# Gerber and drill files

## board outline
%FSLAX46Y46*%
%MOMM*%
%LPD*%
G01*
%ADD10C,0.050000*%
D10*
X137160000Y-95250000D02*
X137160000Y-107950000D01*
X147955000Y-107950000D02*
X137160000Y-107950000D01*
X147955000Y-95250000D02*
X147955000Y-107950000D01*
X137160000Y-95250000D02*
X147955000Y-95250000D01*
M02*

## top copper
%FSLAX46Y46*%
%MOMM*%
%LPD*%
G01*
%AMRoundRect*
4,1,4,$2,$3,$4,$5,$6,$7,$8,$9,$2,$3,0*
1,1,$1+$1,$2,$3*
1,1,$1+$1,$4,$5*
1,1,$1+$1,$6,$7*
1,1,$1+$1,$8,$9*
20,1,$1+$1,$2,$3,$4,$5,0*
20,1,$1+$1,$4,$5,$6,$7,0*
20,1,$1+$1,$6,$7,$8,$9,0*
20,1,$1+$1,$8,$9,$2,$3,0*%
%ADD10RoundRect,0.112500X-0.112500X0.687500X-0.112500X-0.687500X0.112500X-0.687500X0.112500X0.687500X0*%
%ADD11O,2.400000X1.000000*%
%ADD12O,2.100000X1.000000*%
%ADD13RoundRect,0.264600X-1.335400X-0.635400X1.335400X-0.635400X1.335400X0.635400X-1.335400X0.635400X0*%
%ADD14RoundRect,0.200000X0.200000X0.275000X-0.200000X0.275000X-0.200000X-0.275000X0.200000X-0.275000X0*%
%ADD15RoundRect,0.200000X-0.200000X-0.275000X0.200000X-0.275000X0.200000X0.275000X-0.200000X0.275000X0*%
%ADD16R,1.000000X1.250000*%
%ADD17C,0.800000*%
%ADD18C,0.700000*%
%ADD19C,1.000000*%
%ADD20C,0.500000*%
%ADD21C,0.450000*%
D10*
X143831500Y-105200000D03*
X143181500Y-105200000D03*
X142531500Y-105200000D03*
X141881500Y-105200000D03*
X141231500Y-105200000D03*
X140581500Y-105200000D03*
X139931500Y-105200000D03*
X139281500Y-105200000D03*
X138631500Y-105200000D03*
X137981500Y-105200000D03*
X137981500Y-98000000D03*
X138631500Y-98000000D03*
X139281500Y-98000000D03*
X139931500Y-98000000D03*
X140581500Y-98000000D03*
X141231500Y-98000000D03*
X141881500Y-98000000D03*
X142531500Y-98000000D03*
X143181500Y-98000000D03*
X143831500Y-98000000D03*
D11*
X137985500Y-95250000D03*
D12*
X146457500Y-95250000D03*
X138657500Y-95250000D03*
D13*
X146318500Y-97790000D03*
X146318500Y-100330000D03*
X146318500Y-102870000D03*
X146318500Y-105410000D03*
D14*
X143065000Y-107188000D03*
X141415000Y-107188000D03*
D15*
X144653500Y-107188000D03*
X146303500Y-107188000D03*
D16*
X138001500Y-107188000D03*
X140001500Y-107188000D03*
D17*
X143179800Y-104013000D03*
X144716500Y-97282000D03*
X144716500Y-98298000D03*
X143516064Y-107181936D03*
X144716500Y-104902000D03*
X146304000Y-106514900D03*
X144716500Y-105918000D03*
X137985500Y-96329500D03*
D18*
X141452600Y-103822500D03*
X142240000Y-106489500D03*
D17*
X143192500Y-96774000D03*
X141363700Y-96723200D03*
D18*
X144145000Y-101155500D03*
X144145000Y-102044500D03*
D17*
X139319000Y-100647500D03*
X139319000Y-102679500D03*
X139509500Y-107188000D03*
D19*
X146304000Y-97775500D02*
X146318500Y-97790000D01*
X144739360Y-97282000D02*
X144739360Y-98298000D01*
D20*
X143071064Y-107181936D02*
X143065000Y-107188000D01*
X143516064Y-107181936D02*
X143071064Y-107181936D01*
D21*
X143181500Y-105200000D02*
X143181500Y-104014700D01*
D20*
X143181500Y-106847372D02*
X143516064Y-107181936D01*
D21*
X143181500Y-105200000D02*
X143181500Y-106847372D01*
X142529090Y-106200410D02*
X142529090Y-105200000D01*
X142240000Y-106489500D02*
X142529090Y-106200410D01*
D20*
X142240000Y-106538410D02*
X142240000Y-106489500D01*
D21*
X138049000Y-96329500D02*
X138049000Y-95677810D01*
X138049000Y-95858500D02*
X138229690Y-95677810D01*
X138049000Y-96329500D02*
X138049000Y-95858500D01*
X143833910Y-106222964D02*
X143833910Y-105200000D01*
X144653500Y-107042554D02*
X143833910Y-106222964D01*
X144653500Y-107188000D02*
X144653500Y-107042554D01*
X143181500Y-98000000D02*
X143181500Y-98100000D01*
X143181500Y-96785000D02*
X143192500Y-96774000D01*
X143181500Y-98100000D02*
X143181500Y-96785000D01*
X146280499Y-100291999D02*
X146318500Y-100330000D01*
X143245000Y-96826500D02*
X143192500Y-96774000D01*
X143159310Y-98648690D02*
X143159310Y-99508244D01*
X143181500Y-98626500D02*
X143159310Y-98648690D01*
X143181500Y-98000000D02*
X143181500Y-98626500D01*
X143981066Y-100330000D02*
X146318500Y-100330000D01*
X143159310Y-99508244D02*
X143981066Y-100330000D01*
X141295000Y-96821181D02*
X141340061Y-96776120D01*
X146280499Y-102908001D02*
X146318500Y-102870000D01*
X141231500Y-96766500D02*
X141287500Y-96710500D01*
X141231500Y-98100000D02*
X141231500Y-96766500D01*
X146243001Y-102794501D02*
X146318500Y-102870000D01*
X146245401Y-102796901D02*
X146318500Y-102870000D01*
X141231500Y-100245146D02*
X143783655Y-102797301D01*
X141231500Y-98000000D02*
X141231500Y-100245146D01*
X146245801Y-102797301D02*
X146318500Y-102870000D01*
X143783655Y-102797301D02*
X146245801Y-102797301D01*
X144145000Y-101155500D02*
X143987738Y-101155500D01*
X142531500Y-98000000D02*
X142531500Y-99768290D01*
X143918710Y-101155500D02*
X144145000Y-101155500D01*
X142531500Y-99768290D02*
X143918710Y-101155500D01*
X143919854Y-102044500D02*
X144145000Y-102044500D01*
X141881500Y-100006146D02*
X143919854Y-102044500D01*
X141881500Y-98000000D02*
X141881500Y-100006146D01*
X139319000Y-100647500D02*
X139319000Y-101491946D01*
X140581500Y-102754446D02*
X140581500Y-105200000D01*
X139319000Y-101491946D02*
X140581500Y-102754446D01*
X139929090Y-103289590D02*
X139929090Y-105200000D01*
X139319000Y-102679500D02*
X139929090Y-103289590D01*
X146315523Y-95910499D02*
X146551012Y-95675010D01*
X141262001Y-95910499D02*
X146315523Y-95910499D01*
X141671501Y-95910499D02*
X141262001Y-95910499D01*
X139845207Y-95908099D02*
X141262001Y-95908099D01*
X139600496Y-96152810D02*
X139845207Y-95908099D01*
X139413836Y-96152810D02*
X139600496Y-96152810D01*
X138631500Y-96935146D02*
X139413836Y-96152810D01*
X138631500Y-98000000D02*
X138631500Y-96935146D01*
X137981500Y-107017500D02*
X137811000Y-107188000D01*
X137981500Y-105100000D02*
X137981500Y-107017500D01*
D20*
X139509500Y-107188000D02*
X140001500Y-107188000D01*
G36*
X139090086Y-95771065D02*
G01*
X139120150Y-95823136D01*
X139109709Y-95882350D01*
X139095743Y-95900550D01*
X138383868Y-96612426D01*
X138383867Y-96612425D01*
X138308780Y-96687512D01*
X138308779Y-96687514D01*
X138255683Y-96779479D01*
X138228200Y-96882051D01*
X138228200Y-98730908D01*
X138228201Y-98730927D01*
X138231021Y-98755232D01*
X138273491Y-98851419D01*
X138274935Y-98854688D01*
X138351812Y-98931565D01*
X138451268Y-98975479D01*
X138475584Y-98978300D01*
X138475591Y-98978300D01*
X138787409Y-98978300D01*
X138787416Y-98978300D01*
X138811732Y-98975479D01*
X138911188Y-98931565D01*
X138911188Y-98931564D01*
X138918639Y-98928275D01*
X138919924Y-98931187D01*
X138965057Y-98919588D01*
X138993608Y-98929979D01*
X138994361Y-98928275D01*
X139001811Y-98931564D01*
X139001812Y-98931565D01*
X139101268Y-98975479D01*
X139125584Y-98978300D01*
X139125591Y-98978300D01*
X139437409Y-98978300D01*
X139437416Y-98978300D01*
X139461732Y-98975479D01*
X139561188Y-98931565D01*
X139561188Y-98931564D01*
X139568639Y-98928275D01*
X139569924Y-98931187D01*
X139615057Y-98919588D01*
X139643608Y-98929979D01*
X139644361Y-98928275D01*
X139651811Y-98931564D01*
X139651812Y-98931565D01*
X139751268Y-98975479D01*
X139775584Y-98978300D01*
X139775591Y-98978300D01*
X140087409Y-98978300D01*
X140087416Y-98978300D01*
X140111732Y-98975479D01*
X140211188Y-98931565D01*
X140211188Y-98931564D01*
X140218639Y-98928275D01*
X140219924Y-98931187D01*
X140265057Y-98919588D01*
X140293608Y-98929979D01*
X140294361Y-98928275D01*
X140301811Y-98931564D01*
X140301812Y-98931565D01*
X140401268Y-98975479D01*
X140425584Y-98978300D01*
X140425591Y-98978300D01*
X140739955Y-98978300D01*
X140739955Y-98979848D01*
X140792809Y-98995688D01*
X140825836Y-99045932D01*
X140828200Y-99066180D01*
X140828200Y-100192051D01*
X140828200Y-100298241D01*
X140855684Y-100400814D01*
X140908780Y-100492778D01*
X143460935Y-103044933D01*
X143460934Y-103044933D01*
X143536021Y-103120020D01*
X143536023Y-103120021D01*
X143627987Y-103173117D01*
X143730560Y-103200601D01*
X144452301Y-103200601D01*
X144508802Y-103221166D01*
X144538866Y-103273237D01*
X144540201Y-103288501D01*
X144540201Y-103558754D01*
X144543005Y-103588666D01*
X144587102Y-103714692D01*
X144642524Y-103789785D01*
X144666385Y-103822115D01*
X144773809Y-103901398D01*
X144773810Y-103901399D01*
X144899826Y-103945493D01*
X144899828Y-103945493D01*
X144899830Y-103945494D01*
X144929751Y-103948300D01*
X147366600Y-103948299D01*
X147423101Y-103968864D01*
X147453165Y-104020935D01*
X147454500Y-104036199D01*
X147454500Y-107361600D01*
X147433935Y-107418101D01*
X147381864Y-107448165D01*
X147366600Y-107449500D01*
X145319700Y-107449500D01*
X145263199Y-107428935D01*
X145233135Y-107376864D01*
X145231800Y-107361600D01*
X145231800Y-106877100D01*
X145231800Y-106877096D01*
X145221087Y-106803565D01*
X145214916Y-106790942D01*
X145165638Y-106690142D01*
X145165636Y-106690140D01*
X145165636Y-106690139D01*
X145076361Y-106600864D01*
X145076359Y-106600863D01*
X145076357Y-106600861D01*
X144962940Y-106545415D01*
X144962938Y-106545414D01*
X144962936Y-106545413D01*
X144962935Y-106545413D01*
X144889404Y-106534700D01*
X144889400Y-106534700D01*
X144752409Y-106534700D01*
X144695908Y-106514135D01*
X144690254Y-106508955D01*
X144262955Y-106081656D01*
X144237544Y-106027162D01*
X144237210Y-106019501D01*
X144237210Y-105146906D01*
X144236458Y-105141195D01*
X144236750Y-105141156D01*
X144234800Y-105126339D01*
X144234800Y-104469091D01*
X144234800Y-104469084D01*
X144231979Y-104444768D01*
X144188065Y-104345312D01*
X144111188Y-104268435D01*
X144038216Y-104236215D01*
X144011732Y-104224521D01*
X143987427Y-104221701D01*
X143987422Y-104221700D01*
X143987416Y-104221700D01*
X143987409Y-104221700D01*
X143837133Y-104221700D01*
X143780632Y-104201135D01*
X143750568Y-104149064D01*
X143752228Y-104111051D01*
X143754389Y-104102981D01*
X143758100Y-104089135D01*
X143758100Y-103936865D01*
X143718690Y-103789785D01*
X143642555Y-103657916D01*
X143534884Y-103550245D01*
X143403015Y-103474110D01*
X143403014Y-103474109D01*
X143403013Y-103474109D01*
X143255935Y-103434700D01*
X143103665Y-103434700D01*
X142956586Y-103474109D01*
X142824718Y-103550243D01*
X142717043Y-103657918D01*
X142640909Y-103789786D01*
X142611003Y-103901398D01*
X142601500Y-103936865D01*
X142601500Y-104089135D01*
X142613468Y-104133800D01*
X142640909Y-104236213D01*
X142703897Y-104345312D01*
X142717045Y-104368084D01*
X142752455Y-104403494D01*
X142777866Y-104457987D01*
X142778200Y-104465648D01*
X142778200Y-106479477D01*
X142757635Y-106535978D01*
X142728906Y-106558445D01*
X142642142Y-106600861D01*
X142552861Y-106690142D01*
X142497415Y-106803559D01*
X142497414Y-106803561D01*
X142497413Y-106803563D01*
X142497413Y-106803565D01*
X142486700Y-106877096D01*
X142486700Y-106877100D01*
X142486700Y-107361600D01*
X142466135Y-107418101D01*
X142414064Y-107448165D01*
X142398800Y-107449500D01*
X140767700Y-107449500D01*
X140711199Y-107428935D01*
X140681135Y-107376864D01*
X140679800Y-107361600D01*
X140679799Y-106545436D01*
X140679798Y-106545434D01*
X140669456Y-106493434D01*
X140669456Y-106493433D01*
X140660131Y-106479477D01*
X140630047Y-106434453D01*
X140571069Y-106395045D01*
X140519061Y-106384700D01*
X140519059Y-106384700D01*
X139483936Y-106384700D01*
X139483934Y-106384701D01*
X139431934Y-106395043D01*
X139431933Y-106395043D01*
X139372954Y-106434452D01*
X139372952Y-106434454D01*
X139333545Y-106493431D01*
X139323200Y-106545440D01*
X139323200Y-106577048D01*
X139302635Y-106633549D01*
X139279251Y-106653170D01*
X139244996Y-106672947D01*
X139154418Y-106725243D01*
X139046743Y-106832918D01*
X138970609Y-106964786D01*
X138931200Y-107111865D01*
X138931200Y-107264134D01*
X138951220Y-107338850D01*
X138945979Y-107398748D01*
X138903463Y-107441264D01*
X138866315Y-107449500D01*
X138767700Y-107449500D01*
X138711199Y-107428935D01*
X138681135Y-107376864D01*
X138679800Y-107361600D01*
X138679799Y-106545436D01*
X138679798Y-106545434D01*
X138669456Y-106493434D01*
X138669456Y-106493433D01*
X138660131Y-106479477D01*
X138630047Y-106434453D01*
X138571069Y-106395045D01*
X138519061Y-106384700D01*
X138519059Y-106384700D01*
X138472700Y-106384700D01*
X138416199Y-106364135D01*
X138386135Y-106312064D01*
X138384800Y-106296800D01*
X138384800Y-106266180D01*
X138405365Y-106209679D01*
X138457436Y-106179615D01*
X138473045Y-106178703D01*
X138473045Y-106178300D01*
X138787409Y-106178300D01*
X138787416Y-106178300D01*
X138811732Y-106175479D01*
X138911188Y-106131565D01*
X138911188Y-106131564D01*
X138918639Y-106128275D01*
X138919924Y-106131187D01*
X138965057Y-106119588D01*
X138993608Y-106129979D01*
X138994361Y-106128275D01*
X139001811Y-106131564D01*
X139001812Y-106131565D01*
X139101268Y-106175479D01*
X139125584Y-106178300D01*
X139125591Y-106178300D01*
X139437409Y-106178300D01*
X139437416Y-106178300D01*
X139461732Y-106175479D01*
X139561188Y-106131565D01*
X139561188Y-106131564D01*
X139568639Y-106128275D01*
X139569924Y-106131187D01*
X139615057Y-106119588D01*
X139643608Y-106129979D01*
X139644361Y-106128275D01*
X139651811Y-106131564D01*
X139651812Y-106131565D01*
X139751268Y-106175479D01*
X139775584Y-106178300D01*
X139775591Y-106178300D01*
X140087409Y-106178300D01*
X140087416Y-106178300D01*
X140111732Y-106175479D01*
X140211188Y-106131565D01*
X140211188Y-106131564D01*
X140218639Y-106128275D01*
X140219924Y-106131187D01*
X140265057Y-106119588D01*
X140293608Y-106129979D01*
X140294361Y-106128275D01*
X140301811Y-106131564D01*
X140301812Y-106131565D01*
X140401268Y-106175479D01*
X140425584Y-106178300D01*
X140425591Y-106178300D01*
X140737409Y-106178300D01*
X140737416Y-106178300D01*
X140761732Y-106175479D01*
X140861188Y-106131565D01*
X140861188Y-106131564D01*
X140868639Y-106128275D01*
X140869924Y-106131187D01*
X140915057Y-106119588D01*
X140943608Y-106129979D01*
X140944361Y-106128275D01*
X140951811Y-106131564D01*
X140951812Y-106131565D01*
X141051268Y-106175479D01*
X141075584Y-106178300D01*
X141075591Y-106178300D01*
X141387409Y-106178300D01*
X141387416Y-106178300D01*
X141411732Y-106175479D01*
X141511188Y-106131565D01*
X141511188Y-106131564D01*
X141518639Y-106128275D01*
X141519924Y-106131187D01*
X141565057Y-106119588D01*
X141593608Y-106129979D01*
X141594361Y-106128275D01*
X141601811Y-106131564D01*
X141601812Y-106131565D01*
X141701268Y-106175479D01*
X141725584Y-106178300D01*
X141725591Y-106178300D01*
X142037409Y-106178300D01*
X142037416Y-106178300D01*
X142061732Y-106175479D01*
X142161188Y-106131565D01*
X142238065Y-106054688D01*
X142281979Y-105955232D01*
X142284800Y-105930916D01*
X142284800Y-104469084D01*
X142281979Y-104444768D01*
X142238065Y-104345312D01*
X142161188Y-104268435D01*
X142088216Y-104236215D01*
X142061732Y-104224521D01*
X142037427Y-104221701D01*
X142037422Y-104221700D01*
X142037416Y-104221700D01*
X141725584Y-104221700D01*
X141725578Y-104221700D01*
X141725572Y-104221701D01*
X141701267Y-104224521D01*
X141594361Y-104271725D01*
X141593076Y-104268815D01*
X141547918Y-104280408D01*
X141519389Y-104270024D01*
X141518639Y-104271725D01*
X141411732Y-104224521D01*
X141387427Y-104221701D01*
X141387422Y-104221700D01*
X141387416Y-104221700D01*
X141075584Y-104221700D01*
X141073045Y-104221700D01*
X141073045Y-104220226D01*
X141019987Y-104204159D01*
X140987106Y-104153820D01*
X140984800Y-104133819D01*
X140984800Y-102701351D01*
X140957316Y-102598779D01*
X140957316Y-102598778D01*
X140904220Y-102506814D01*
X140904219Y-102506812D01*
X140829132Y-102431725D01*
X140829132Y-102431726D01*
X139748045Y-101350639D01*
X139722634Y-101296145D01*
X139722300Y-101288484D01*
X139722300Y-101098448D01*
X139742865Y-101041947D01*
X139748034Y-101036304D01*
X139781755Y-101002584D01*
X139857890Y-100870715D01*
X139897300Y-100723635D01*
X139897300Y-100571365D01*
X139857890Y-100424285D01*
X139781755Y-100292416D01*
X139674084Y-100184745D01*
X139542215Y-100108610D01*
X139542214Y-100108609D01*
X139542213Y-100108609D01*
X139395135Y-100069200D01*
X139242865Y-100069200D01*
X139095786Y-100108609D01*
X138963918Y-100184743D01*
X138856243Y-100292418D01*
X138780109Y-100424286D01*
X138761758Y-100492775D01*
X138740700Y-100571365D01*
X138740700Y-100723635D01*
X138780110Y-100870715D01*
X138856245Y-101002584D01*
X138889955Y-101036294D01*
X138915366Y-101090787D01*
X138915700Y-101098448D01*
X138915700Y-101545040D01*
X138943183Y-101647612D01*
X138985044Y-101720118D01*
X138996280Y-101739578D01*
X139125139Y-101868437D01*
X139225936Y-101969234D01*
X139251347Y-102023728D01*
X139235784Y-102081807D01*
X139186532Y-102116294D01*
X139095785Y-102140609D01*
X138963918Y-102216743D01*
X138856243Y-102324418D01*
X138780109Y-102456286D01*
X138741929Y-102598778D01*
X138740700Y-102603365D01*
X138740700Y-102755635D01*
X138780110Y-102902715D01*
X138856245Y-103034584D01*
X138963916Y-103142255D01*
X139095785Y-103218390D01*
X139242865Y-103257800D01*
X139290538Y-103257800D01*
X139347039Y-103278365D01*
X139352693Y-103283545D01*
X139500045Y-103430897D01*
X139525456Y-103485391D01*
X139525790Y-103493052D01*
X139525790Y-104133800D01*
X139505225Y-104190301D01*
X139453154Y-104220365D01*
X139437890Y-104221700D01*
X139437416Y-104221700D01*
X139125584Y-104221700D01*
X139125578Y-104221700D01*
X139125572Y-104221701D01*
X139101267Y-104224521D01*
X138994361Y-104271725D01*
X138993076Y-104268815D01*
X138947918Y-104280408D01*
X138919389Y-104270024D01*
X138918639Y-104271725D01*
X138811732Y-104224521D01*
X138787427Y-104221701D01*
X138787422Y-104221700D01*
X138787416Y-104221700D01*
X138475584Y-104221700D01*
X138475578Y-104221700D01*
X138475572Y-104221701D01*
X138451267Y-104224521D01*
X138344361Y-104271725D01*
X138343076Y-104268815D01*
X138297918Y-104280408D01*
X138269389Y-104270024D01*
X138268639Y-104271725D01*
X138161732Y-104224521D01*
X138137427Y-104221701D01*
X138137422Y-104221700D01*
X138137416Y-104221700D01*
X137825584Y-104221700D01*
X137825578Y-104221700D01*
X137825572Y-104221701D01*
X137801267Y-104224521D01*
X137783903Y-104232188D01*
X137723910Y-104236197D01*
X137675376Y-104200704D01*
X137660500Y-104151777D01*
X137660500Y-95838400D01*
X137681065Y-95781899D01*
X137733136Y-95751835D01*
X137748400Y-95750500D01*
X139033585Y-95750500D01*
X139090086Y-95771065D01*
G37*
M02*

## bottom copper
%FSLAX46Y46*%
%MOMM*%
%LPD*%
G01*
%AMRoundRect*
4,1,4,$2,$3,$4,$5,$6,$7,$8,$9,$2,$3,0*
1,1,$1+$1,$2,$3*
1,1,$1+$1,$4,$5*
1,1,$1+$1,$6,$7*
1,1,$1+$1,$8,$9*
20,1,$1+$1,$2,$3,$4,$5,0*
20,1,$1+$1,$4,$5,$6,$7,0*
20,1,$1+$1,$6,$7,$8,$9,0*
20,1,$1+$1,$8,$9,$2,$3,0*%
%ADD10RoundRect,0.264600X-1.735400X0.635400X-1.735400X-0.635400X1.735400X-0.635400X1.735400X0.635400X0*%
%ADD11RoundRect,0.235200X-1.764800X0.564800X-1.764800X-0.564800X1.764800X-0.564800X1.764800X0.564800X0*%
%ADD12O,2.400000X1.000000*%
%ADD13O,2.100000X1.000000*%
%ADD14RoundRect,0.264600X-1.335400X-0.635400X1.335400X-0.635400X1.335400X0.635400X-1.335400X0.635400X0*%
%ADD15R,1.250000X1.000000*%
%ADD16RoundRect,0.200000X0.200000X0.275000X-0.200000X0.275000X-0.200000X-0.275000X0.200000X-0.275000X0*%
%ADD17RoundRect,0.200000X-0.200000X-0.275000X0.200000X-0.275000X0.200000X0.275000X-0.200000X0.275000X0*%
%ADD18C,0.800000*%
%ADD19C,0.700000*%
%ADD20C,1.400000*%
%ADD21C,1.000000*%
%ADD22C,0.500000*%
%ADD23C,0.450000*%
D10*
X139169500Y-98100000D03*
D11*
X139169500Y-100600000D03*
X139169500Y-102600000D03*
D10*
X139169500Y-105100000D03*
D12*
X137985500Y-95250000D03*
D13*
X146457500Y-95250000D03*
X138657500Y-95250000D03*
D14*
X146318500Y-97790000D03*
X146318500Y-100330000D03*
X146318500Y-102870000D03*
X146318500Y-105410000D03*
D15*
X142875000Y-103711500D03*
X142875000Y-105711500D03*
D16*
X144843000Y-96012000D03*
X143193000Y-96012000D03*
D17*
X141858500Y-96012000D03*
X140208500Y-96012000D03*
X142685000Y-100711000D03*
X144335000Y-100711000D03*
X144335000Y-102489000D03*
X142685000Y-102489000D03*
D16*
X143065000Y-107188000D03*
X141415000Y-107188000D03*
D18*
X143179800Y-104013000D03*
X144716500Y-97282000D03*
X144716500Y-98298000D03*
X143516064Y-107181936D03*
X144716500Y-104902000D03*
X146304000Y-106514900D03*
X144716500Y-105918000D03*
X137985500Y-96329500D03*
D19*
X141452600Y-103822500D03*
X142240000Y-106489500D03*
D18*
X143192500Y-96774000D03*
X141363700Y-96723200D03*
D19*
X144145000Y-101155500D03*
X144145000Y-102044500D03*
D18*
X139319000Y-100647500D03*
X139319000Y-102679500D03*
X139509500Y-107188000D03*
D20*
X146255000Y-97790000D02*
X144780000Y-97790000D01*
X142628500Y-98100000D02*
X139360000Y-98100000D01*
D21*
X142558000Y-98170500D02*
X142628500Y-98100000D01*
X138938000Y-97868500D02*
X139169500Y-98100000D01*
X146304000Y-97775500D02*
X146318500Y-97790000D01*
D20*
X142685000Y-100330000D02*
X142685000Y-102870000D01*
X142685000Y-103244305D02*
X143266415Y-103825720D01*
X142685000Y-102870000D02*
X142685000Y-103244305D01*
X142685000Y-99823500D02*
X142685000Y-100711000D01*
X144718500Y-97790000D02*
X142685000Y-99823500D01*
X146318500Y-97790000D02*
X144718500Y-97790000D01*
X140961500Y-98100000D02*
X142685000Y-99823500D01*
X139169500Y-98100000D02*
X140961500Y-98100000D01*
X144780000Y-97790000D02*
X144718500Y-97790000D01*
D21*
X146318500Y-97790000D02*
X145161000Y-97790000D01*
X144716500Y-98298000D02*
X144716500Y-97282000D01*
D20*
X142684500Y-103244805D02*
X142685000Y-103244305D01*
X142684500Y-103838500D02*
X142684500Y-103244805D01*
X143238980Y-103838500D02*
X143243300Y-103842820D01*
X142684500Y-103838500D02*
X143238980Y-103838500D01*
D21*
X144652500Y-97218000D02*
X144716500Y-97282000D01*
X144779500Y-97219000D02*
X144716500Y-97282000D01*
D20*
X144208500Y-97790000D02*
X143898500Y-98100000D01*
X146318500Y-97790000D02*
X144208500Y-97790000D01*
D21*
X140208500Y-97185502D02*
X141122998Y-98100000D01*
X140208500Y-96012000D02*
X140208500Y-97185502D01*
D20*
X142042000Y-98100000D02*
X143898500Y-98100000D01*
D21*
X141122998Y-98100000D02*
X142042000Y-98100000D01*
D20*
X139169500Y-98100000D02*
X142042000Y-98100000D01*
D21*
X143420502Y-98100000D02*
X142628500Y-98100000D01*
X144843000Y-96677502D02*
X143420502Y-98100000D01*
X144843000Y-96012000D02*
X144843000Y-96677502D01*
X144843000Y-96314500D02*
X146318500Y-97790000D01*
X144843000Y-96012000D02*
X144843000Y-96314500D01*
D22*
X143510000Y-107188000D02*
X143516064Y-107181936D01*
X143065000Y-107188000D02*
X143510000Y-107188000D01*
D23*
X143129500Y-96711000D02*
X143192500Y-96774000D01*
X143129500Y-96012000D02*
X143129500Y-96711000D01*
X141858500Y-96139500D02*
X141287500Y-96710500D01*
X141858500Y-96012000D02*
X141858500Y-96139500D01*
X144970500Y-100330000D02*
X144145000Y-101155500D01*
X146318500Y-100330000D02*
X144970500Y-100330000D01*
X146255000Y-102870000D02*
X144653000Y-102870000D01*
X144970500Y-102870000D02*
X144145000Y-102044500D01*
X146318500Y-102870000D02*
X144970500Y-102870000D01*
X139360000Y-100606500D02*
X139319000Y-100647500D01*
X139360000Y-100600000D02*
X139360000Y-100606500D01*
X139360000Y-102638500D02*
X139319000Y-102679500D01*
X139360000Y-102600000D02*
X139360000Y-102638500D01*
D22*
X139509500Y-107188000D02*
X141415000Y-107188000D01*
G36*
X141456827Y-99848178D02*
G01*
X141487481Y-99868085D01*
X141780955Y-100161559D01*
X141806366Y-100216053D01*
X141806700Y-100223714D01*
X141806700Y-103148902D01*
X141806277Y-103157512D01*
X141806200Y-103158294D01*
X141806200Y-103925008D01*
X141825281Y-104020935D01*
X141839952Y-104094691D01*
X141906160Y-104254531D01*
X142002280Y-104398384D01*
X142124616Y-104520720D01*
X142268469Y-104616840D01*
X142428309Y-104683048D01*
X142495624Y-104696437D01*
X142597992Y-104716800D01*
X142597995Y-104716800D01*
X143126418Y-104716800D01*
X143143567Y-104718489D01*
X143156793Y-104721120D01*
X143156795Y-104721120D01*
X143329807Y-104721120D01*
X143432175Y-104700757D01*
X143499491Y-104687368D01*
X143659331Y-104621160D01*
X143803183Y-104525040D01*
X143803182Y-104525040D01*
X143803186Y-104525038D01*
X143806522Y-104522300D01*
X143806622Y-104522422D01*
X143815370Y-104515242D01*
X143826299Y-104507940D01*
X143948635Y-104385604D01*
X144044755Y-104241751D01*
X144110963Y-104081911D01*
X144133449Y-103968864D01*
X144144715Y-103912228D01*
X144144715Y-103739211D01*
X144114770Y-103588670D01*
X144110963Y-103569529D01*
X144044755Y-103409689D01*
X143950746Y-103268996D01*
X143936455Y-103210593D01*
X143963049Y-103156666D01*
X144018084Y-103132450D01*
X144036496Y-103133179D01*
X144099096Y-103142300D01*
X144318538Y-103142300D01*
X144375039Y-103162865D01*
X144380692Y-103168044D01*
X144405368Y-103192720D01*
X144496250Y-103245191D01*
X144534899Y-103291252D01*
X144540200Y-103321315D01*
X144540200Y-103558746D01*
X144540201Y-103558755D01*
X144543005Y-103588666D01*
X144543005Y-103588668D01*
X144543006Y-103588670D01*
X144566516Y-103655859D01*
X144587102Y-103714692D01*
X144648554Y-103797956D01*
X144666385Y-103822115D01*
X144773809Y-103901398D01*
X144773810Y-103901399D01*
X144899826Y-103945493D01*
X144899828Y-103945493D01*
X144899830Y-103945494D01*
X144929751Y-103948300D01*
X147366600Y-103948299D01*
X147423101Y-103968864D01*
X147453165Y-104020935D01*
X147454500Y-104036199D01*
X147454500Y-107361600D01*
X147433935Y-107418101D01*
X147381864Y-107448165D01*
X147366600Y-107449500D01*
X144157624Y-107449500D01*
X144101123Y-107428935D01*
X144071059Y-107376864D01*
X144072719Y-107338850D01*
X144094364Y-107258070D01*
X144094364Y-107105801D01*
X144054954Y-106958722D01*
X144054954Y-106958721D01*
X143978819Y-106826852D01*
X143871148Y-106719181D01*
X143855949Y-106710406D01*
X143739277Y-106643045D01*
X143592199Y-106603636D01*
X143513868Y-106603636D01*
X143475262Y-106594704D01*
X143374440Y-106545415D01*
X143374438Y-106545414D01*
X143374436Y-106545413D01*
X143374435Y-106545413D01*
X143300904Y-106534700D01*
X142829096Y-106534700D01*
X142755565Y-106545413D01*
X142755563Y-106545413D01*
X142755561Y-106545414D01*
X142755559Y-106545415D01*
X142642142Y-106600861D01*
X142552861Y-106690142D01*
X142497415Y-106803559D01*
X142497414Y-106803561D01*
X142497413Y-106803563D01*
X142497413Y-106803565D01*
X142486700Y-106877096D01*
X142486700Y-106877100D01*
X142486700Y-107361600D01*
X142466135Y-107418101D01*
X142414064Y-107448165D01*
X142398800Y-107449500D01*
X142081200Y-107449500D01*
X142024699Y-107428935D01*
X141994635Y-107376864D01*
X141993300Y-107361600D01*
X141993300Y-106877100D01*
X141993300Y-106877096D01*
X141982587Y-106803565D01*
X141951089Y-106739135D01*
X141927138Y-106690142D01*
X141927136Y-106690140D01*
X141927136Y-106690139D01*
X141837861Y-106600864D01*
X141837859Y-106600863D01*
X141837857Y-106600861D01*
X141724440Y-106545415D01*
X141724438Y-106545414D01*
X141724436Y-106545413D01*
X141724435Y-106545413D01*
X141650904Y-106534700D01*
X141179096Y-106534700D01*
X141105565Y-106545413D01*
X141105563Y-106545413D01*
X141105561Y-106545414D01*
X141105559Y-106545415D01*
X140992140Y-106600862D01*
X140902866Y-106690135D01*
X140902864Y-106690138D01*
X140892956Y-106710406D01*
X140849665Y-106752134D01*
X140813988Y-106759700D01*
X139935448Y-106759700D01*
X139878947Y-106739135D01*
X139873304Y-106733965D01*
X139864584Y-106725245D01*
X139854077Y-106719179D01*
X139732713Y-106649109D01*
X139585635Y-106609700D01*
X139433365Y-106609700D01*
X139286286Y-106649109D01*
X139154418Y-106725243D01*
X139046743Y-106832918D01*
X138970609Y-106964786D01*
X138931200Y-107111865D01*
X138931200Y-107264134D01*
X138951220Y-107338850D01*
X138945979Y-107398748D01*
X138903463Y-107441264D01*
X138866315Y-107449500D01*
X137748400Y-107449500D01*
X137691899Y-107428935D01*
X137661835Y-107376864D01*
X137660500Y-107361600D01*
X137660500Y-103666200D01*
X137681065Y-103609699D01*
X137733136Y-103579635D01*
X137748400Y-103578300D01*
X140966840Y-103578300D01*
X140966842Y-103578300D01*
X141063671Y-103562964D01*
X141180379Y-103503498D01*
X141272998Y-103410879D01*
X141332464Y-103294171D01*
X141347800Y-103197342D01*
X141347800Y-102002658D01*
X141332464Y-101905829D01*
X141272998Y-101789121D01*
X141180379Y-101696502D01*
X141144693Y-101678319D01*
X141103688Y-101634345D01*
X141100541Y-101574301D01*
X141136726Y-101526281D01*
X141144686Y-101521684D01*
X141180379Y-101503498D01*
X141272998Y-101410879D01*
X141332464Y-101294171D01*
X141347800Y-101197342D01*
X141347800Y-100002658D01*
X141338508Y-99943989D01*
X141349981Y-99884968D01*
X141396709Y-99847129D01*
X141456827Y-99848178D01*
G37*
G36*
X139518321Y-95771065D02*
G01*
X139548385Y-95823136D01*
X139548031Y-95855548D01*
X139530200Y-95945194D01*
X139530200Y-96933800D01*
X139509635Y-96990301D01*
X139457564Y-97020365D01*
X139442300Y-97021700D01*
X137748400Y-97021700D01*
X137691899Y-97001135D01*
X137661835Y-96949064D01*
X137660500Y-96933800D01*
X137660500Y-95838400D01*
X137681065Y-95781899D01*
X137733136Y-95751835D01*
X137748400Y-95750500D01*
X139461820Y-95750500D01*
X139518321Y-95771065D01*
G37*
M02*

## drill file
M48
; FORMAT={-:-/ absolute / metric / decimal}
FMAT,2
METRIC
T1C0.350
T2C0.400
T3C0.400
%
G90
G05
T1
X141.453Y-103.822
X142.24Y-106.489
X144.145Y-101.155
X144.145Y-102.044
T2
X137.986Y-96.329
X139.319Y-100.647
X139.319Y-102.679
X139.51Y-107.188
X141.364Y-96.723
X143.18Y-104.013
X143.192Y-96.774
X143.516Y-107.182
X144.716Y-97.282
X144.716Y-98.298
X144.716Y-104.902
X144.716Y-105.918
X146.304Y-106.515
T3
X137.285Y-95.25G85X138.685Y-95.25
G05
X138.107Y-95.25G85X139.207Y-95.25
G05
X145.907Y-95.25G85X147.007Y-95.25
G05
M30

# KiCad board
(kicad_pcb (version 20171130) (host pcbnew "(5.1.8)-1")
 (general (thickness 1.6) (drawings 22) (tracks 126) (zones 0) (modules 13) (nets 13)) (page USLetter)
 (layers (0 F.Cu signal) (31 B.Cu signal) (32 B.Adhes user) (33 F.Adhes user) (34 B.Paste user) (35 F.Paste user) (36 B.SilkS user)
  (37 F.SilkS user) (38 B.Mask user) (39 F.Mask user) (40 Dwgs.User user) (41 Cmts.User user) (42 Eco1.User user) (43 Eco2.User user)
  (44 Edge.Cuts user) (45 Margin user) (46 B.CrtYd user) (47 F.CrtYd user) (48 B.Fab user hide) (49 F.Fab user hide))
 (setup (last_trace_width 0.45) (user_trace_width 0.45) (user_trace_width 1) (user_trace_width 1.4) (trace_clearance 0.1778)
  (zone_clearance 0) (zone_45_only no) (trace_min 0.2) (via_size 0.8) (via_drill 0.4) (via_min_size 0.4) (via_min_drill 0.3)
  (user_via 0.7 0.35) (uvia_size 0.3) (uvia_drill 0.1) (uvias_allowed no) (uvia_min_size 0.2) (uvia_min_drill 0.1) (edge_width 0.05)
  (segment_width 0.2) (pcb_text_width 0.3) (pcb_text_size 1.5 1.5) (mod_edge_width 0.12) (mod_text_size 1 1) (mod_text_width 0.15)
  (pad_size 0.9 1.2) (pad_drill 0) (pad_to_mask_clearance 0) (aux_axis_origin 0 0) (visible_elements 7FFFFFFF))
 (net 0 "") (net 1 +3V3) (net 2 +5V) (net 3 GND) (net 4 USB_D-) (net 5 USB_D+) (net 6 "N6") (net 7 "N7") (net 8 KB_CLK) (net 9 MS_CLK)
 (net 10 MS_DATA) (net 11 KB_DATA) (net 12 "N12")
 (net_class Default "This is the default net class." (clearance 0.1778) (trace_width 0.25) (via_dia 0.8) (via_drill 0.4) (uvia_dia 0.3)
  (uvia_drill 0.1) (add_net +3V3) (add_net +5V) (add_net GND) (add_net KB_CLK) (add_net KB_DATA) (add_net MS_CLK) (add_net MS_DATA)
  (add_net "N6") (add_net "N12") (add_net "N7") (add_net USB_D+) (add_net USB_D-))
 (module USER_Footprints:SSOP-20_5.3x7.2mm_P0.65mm (layer F.Cu) (at 140.9065 101.6 270)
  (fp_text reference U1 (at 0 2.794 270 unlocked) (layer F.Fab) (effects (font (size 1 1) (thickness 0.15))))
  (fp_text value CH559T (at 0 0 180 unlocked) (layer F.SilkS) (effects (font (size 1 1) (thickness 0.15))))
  (pad 20 smd roundrect (at 3.6 -2.925 270) (size 1.6 0.45) (layers F.Cu F.Paste F.Mask) (roundrect_rratio 0.25) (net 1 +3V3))
  (pad 19 smd roundrect (at 3.6 -2.275 270) (size 1.6 0.45) (layers F.Cu F.Paste F.Mask) (roundrect_rratio 0.25) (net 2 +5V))
  (pad 18 smd roundrect (at 3.6 -1.625 270) (size 1.6 0.45) (layers F.Cu F.Paste F.Mask) (roundrect_rratio 0.25) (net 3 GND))
  (pad 17 smd roundrect (at 3.6 -0.975 270) (size 1.6 0.45) (layers F.Cu F.Paste F.Mask) (roundrect_rratio 0.25))
  (pad 16 smd roundrect (at 3.6 -0.325 270) (size 1.6 0.45) (layers F.Cu F.Paste F.Mask) (roundrect_rratio 0.25))
  (pad 15 smd roundrect (at 3.6 0.325 270) (size 1.6 0.45) (layers F.Cu F.Paste F.Mask) (roundrect_rratio 0.25) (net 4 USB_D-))
  (pad 14 smd roundrect (at 3.6 0.975 270) (size 1.6 0.45) (layers F.Cu F.Paste F.Mask) (roundrect_rratio 0.25) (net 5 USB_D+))
  (pad 13 smd roundrect (at 3.6 1.625 270) (size 1.6 0.45) (layers F.Cu F.Paste F.Mask) (roundrect_rratio 0.25))
  (pad 12 smd roundrect (at 3.6 2.275 270) (size 1.6 0.45) (layers F.Cu F.Paste F.Mask) (roundrect_rratio 0.25))
  (pad 11 smd roundrect (at 3.6 2.925 270) (size 1.6 0.45) (layers F.Cu F.Paste F.Mask) (roundrect_rratio 0.25) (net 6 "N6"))
  (pad 10 smd roundrect (at -3.6 2.925 270) (size 1.6 0.45) (layers F.Cu F.Paste F.Mask) (roundrect_rratio 0.25) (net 3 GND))
  (pad 9 smd roundrect (at -3.6 2.275 270) (size 1.6 0.45) (layers F.Cu F.Paste F.Mask) (roundrect_rratio 0.25) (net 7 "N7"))
  (pad 8 smd roundrect (at -3.6 1.625 270) (size 1.6 0.45) (layers F.Cu F.Paste F.Mask) (roundrect_rratio 0.25))
  (pad 7 smd roundrect (at -3.6 0.975 270) (size 1.6 0.45) (layers F.Cu F.Paste F.Mask) (roundrect_rratio 0.25))
  (pad 6 smd roundrect (at -3.6 0.325 270) (size 1.6 0.45) (layers F.Cu F.Paste F.Mask) (roundrect_rratio 0.25))
  (pad 5 smd roundrect (at -3.6 -0.325 270) (size 1.6 0.45) (layers F.Cu F.Paste F.Mask) (roundrect_rratio 0.25) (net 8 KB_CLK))
  (pad 4 smd roundrect (at -3.6 -0.975 270) (size 1.6 0.45) (layers F.Cu F.Paste F.Mask) (roundrect_rratio 0.25) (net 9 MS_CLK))
  (pad 3 smd roundrect (at -3.6 -1.625 270) (size 1.6 0.45) (layers F.Cu F.Paste F.Mask) (roundrect_rratio 0.25) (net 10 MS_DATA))
  (pad 2 smd roundrect (at -3.6 -2.275 270) (size 1.6 0.45) (layers F.Cu F.Paste F.Mask) (roundrect_rratio 0.25) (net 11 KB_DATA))
  (pad 1 smd roundrect (at -3.6 -2.925 270) (size 1.6 0.45) (layers F.Cu F.Paste F.Mask) (roundrect_rratio 0.25)))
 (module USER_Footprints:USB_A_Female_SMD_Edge (layer F.Cu) (at 136.9695 101.6 270)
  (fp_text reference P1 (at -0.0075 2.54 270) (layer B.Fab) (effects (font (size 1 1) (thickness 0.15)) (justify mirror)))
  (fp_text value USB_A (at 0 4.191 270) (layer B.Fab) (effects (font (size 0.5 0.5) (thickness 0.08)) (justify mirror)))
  (pad 1 smd roundrect (at -3.5 -2.2 270) (size 1.8 4) (layers B.Cu B.Paste B.Mask) (roundrect_rratio 0.147) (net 2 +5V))
  (pad 2 smd roundrect (at -1 -2.2 270) (size 1.6 4) (layers B.Cu B.Paste B.Mask) (roundrect_rratio 0.147) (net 4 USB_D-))
  (pad 3 smd roundrect (at 1 -2.2 270) (size 1.6 4) (layers B.Cu B.Paste B.Mask) (roundrect_rratio 0.147) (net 5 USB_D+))
  (pad 4 smd roundrect (at 3.5 -2.2 270) (size 1.8 4) (layers B.Cu B.Paste B.Mask) (roundrect_rratio 0.147) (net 3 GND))
  (pad 4 thru_hole oval (at -6.35 -1.016) (size 2.4 1) (drill oval 1.8 0.4) (layers *.Cu *.Mask) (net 3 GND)))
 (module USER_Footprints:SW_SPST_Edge (layer F.Cu) (at 142.5575 95.25)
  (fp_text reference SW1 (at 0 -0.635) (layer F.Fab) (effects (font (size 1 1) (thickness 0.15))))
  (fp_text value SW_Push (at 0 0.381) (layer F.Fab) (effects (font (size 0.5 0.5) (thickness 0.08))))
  (pad 2 thru_hole oval (at 3.9 0) (size 2.1 1) (drill oval 1.5 0.4) (layers *.Cu *.Mask) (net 7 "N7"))
  (pad 1 thru_hole oval (at -3.9 0) (size 2.1 1) (drill oval 1.5 0.4) (layers *.Cu *.Mask) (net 3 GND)))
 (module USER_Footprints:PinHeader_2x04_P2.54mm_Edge (layer F.Cu) (at 148.0185 97.79)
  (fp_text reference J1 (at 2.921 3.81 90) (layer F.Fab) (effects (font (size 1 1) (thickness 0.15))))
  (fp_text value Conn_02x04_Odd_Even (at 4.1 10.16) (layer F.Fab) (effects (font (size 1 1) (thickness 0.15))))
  (pad 1 smd roundrect (at -1.7 0) (size 3.2 1.8) (layers F.Cu F.Paste F.Mask) (roundrect_rratio 0.147) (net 2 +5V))
  (pad 2 smd roundrect (at -1.7 0) (size 3.2 1.8) (layers B.Cu B.Paste B.Mask) (roundrect_rratio 0.147) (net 2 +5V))
  (pad 3 smd roundrect (at -1.7 2.54) (size 3.2 1.8) (layers F.Cu F.Paste F.Mask) (roundrect_rratio 0.147) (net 11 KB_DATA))
  (pad 4 smd roundrect (at -1.7 2.54) (size 3.2 1.8) (layers B.Cu B.Paste B.Mask) (roundrect_rratio 0.147) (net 10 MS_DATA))
  (pad 5 smd roundrect (at -1.7 5.08) (size 3.2 1.8) (layers F.Cu F.Paste F.Mask) (roundrect_rratio 0.147) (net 8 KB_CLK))
  (pad 6 smd roundrect (at -1.7 5.08) (size 3.2 1.8) (layers B.Cu B.Paste B.Mask) (roundrect_rratio 0.147) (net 9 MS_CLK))
  (pad 7 smd roundrect (at -1.7 7.62) (size 3.2 1.8) (layers F.Cu F.Paste F.Mask) (roundrect_rratio 0.147) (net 3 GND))
  (pad 8 smd roundrect (at -1.7 7.62) (size 3.2 1.8) (layers B.Cu B.Paste B.Mask) (roundrect_rratio 0.147) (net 3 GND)))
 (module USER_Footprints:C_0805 (layer B.Cu) (at 142.875 104.7115 270)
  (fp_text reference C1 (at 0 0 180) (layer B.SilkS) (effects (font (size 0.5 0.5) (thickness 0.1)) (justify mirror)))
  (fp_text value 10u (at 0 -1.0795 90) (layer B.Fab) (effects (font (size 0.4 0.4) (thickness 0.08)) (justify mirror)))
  (pad 1 smd rect (at -1 0 270) (size 1 1.25) (layers B.Cu B.Paste B.Mask) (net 2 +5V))
  (pad 2 smd rect (at 1 0 270) (size 1 1.25) (layers B.Cu B.Paste B.Mask) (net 3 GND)))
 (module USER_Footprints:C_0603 (layer F.Cu) (at 142.24 107.188 180)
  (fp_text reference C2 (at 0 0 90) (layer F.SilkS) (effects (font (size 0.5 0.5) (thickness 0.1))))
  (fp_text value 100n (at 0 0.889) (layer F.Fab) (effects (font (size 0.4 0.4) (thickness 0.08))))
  (pad 1 smd roundrect (at -0.825 0 180) (size 0.8 0.95) (layers F.Cu F.Paste F.Mask) (roundrect_rratio 0.25) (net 2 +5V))
  (pad 2 smd roundrect (at 0.825 0 180) (size 0.8 0.95) (layers F.Cu F.Paste F.Mask) (roundrect_rratio 0.25) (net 3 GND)))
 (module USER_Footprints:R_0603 (layer B.Cu) (at 144.018 96.012 180)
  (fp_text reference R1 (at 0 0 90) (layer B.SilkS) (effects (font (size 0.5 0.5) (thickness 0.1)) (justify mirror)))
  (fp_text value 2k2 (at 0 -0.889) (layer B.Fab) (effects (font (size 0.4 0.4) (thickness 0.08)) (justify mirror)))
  (pad 1 smd roundrect (at -0.825 0 180) (size 0.8 0.95) (layers B.Cu B.Paste B.Mask) (roundrect_rratio 0.25) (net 2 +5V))
  (pad 2 smd roundrect (at 0.825 0 180) (size 0.8 0.95) (layers B.Cu B.Paste B.Mask) (roundrect_rratio 0.25) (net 11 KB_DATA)))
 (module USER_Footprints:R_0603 (layer B.Cu) (at 141.0335 96.012)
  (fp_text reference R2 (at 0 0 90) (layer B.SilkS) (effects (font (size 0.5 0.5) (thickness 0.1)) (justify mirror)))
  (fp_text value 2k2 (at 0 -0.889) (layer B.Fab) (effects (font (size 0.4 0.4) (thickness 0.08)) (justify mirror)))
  (pad 2 smd roundrect (at 0.825 0) (size 0.8 0.95) (layers B.Cu B.Paste B.Mask) (roundrect_rratio 0.25) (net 8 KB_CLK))
  (pad 1 smd roundrect (at -0.825 0) (size 0.8 0.95) (layers B.Cu B.Paste B.Mask) (roundrect_rratio 0.25) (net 2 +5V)))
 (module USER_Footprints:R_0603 (layer B.Cu) (at 143.51 100.711)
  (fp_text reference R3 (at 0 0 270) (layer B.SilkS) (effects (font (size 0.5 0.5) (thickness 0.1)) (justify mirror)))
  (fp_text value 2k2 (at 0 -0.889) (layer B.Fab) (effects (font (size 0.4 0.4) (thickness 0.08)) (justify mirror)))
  (pad 1 smd roundrect (at -0.825 0) (size 0.8 0.95) (layers B.Cu B.Paste B.Mask) (roundrect_rratio 0.25) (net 2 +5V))
  (pad 2 smd roundrect (at 0.825 0) (size 0.8 0.95) (layers B.Cu B.Paste B.Mask) (roundrect_rratio 0.25) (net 10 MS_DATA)))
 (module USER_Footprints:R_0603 (layer B.Cu) (at 143.51 102.489)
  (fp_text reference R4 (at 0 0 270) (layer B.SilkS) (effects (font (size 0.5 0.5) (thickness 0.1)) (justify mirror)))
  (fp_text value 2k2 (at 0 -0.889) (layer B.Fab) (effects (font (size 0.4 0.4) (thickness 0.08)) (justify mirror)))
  (pad 2 smd roundrect (at 0.825 0) (size 0.8 0.95) (layers B.Cu B.Paste B.Mask) (roundrect_rratio 0.25) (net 9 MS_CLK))
  (pad 1 smd roundrect (at -0.825 0) (size 0.8 0.95) (layers B.Cu B.Paste B.Mask) (roundrect_rratio 0.25) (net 2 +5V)))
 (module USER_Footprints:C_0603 (layer F.Cu) (at 145.4785 107.188)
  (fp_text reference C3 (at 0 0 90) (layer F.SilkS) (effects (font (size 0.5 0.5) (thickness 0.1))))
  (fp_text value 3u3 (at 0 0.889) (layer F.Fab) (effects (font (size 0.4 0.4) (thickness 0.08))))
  (pad 1 smd roundrect (at -0.825 0) (size 0.8 0.95) (layers F.Cu F.Paste F.Mask) (roundrect_rratio 0.25) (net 1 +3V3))
  (pad 2 smd roundrect (at 0.825 0) (size 0.8 0.95) (layers F.Cu F.Paste F.Mask) (roundrect_rratio 0.25) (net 3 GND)))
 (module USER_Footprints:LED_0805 (layer F.Cu) (at 139.0015 107.188)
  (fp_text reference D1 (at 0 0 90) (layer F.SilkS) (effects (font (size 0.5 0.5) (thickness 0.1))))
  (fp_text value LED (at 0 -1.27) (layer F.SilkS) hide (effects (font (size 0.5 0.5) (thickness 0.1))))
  (pad 1 smd rect (at -1 0) (size 1 1.25) (layers F.Cu F.Paste F.Mask) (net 6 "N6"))
  (pad 2 smd rect (at 1 0) (size 1 1.25) (layers F.Cu F.Paste F.Mask) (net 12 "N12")))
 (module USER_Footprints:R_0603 (layer B.Cu) (at 142.24 107.188 180)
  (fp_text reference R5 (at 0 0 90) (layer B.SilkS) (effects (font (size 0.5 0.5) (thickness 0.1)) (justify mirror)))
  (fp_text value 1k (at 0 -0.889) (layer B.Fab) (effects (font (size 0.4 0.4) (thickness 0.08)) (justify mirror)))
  (pad 1 smd roundrect (at -0.825 0 180) (size 0.8 0.95) (layers B.Cu B.Paste B.Mask) (roundrect_rratio 0.25) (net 2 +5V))
  (pad 2 smd roundrect (at 0.825 0 180) (size 0.8 0.95) (layers B.Cu B.Paste B.Mask) (roundrect_rratio 0.25) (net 12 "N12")))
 (gr_line (start 137.16 95.25) (end 137.16 107.95) (layer Edge.Cuts) (width 0.05))
 (gr_line (start 147.955 107.95) (end 137.16 107.95) (layer Edge.Cuts) (width 0.05))
 (gr_line (start 147.955 95.25) (end 147.955 107.95) (layer Edge.Cuts) (width 0.05))
 (gr_line (start 137.16 95.25) (end 147.955 95.25) (layer Edge.Cuts) (width 0.05))
 (segment (start 146.255 97.79) (end 144.78 97.79) (width 1.4) (layer B.Cu) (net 2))
 (segment (start 142.6285 98.1) (end 139.36 98.1) (width 1.4) (layer B.Cu) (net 2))
 (segment (start 142.558 98.1705) (end 142.6285 98.1) (width 1) (layer B.Cu) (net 2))
 (segment (start 138.938 97.8685) (end 139.1695 98.1) (width 1) (layer B.Cu) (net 2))
 (segment (start 146.304 97.7755) (end 146.3185 97.79) (width 1) (layer F.Cu) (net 2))
 (segment (start 146.304 97.7755) (end 146.3185 97.79) (width 1) (layer B.Cu) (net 2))
 (via (at 143.1798 104.013) (size 0.8) (drill 0.4) (layers F.Cu B.Cu) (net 2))
 (segment (start 142.685 100.33) (end 142.685 102.87) (width 1.4) (layer B.Cu) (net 2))
 (segment (start 142.685 103.244305) (end 143.266415 103.82572) (width 1.4) (layer B.Cu) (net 2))
 (segment (start 142.685 102.87) (end 142.685 103.244305) (width 1.4) (layer B.Cu) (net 2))
 (segment (start 142.685 99.8235) (end 142.685 100.711) (width 1.4) (layer B.Cu) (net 2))
 (segment (start 144.7185 97.79) (end 142.685 99.8235) (width 1.4) (layer B.Cu) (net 2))
 (segment (start 146.3185 97.79) (end 144.7185 97.79) (width 1.4) (layer B.Cu) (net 2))
 (segment (start 140.9615 98.1) (end 142.685 99.8235) (width 1.4) (layer B.Cu) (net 2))
 (segment (start 139.1695 98.1) (end 140.9615 98.1) (width 1.4) (layer B.Cu) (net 2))
 (segment (start 144.78 97.79) (end 144.7185 97.79) (width 1.4) (layer B.Cu) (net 2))
 (via (at 144.7165 97.282) (size 0.8) (drill 0.4) (layers F.Cu B.Cu) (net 2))
 (via (at 144.7165 98.298) (size 0.8) (drill 0.4) (layers F.Cu B.Cu) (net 2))
 (segment (start 146.3185 97.79) (end 145.161 97.79) (width 1) (layer B.Cu) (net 2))
 (segment (start 144.7165 98.298) (end 144.7165 97.282) (width 1) (layer B.Cu) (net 2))
 (segment (start 144.73936 97.282) (end 144.73936 98.298) (width 1) (layer F.Cu) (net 2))
 (segment (start 142.6845 103.244805) (end 142.685 103.244305) (width 1.4) (layer B.Cu) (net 2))
 (segment (start 142.6845 103.8385) (end 142.6845 103.244805) (width 1.4) (layer B.Cu) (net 2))
 (segment (start 143.23898 103.8385) (end 143.2433 103.84282) (width 1.4) (layer B.Cu) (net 2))
 (segment (start 142.6845 103.8385) (end 143.23898 103.8385) (width 1.4) (layer B.Cu) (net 2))
 (segment (start 144.6525 97.218) (end 144.7165 97.282) (width 1) (layer B.Cu) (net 2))
 (segment (start 144.7795 97.219) (end 144.7165 97.282) (width 1) (layer B.Cu) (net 2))
 (segment (start 144.2085 97.79) (end 143.8985 98.1) (width 1.4) (layer B.Cu) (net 2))
 (segment (start 146.3185 97.79) (end 144.2085 97.79) (width 1.4) (layer B.Cu) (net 2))
 (segment (start 140.2085 97.185502) (end 141.122998 98.1) (width 1) (layer B.Cu) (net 2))
 (segment (start 140.2085 96.012) (end 140.2085 97.185502) (width 1) (layer B.Cu) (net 2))
 (segment (start 142.042 98.1) (end 143.8985 98.1) (width 1.4) (layer B.Cu) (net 2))
 (segment (start 141.122998 98.1) (end 142.042 98.1) (width 1) (layer B.Cu) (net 2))
 (segment (start 139.1695 98.1) (end 142.042 98.1) (width 1.4) (layer B.Cu) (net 2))
 (segment (start 143.420502 98.1) (end 142.6285 98.1) (width 1) (layer B.Cu) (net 2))
 (segment (start 144.843 96.677502) (end 143.420502 98.1) (width 1) (layer B.Cu) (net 2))
 (segment (start 144.843 96.012) (end 144.843 96.677502) (width 1) (layer B.Cu) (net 2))
 (segment (start 144.843 96.3145) (end 146.3185 97.79) (width 1) (layer B.Cu) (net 2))
 (segment (start 144.843 96.012) (end 144.843 96.3145) (width 1) (layer B.Cu) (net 2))
 (via (at 143.516064 107.181936) (size 0.8) (drill 0.4) (layers F.Cu B.Cu) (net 2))
 (segment (start 143.51 107.188) (end 143.516064 107.181936) (width 0.5) (layer B.Cu) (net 2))
 (segment (start 143.065 107.188) (end 143.51 107.188) (width 0.5) (layer B.Cu) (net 2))
 (segment (start 143.071064 107.181936) (end 143.065 107.188) (width 0.5) (layer F.Cu) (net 2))
 (segment (start 143.516064 107.181936) (end 143.071064 107.181936) (width 0.5) (layer F.Cu) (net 2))
 (segment (start 143.1815 105.2) (end 143.1815 104.0147) (width 0.45) (layer F.Cu) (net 2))
 (segment (start 143.1815 106.847372) (end 143.516064 107.181936) (width 0.5) (layer F.Cu) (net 2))
 (segment (start 143.1815 105.2) (end 143.1815 106.847372) (width 0.45) (layer F.Cu) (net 2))
 (via (at 144.7165 104.902) (size 0.8) (drill 0.4) (layers F.Cu B.Cu) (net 3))
 (via (at 146.304 106.5149) (size 0.8) (drill 0.4) (layers F.Cu B.Cu) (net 3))
 (via (at 144.7165 105.918) (size 0.8) (drill 0.4) (layers F.Cu B.Cu) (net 3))
 (via (at 137.9855 96.3295) (size 0.8) (drill 0.4) (layers F.Cu B.Cu) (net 3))
 (via (at 141.4526 103.8225) (size 0.7) (drill 0.35) (layers F.Cu B.Cu) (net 3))
 (via (at 142.24 106.4895) (size 0.7) (drill 0.35) (layers F.Cu B.Cu) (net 3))
 (segment (start 142.52909 106.20041) (end 142.52909 105.2) (width 0.45) (layer F.Cu) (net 3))
 (segment (start 142.24 106.4895) (end 142.52909 106.20041) (width 0.45) (layer F.Cu) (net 3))
 (segment (start 142.24 106.53841) (end 142.24 106.4895) (width 0.5) (layer F.Cu) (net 3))
 (segment (start 138.049 96.3295) (end 138.049 95.67781) (width 0.45) (layer F.Cu) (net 3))
 (segment (start 138.049 95.8585) (end 138.22969 95.67781) (width 0.45) (layer F.Cu) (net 3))
 (segment (start 138.049 96.3295) (end 138.049 95.8585) (width 0.45) (layer F.Cu) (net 3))
 (segment (start 143.83391 106.222964) (end 143.83391 105.2) (width 0.45) (layer F.Cu) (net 1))
 (segment (start 144.6535 107.042554) (end 143.83391 106.222964) (width 0.45) (layer F.Cu) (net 1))
 (segment (start 144.6535 107.188) (end 144.6535 107.042554) (width 0.45) (layer F.Cu) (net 1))
 (segment (start 143.1815 98) (end 143.1815 98.1) (width 0.45) (layer F.Cu) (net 11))
 (segment (start 143.1815 96.785) (end 143.1925 96.774) (width 0.45) (layer F.Cu) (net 11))
 (segment (start 143.1815 98.1) (end 143.1815 96.785) (width 0.45) (layer F.Cu) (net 11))
 (segment (start 146.280499 100.291999) (end 146.3185 100.33) (width 0.45) (layer F.Cu) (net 11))
 (segment (start 143.1295 96.711) (end 143.1925 96.774) (width 0.45) (layer B.Cu) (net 11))
 (segment (start 143.245 96.8265) (end 143.1925 96.774) (width 0.45) (layer F.Cu) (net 11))
 (segment (start 143.1295 96.012) (end 143.1295 96.711) (width 0.45) (layer B.Cu) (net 11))
 (via (at 143.1925 96.774) (size 0.8) (drill 0.4) (layers F.Cu B.Cu) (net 11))
 (segment (start 143.15931 98.64869) (end 143.15931 99.508244) (width 0.45) (layer F.Cu) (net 11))
 (segment (start 143.1815 98.6265) (end 143.15931 98.64869) (width 0.45) (layer F.Cu) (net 11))
 (segment (start 143.1815 98) (end 143.1815 98.6265) (width 0.45) (layer F.Cu) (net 11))
 (segment (start 143.981066 100.33) (end 146.3185 100.33) (width 0.45) (layer F.Cu) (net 11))
 (segment (start 143.15931 99.508244) (end 143.981066 100.33) (width 0.45) (layer F.Cu) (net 11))
 (via (at 141.3637 96.7232) (size 0.8) (drill 0.4) (layers F.Cu B.Cu) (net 8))
 (segment (start 141.295 96.821181) (end 141.340061 96.77612) (width 0.45) (layer F.Cu) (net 8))
 (segment (start 146.280499 102.908001) (end 146.3185 102.87) (width 0.45) (layer F.Cu) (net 8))
 (segment (start 141.2315 96.7665) (end 141.2875 96.7105) (width 0.45) (layer F.Cu) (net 8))
 (segment (start 141.2315 98.1) (end 141.2315 96.7665) (width 0.45) (layer F.Cu) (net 8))
 (segment (start 141.8585 96.1395) (end 141.2875 96.7105) (width 0.45) (layer B.Cu) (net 8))
 (segment (start 141.8585 96.012) (end 141.8585 96.1395) (width 0.45) (layer B.Cu) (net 8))
 (segment (start 146.243001 102.794501) (end 146.3185 102.87) (width 0.45) (layer F.Cu) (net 8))
 (segment (start 146.245401 102.796901) (end 146.3185 102.87) (width 0.45) (layer F.Cu) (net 8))
 (segment (start 141.2315 100.245146) (end 143.783655 102.797301) (width 0.45) (layer F.Cu) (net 8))
 (segment (start 141.2315 98) (end 141.2315 100.245146) (width 0.45) (layer F.Cu) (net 8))
 (segment (start 146.245801 102.797301) (end 146.3185 102.87) (width 0.45) (layer F.Cu) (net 8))
 (segment (start 143.783655 102.797301) (end 146.245801 102.797301) (width 0.45) (layer F.Cu) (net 8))
 (via (at 144.145 101.1555) (size 0.7) (drill 0.35) (layers F.Cu B.Cu) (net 10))
 (segment (start 144.145 101.1555) (end 143.987738 101.1555) (width 0.45) (layer F.Cu) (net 10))
 (segment (start 142.5315 98) (end 142.5315 99.76829) (width 0.45) (layer F.Cu) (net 10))
 (segment (start 143.91871 101.1555) (end 144.145 101.1555) (width 0.45) (layer F.Cu) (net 10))
 (segment (start 142.5315 99.76829) (end 143.91871 101.1555) (width 0.45) (layer F.Cu) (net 10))
 (segment (start 144.9705 100.33) (end 144.145 101.1555) (width 0.45) (layer B.Cu) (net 10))
 (segment (start 146.3185 100.33) (end 144.9705 100.33) (width 0.45) (layer B.Cu) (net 10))
 (via (at 144.145 102.0445) (size 0.7) (drill 0.35) (layers F.Cu B.Cu) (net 9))
 (segment (start 146.255 102.87) (end 144.653 102.87) (width 0.45) (layer B.Cu) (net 9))
 (segment (start 143.919854 102.0445) (end 144.145 102.0445) (width 0.45) (layer F.Cu) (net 9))
 (segment (start 141.8815 100.006146) (end 143.919854 102.0445) (width 0.45) (layer F.Cu) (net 9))
 (segment (start 141.8815 98) (end 141.8815 100.006146) (width 0.45) (layer F.Cu) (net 9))
 (segment (start 144.9705 102.87) (end 144.145 102.0445) (width 0.45) (layer B.Cu) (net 9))
 (segment (start 146.3185 102.87) (end 144.9705 102.87) (width 0.45) (layer B.Cu) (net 9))
 (via (at 139.319 100.6475) (size 0.8) (drill 0.4) (layers F.Cu B.Cu) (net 4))
 (segment (start 139.36 100.6065) (end 139.319 100.6475) (width 0.45) (layer B.Cu) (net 4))
 (segment (start 139.36 100.6) (end 139.36 100.6065) (width 0.45) (layer B.Cu) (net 4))
 (segment (start 139.319 100.6475) (end 139.319 101.491946) (width 0.45) (layer F.Cu) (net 4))
 (segment (start 140.5815 102.754446) (end 140.5815 105.2) (width 0.45) (layer F.Cu) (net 4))
 (segment (start 139.319 101.491946) (end 140.5815 102.754446) (width 0.45) (layer F.Cu) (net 4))
 (via (at 139.319 102.6795) (size 0.8) (drill 0.4) (layers F.Cu B.Cu) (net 5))
 (segment (start 139.36 102.6385) (end 139.319 102.6795) (width 0.45) (layer B.Cu) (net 5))
 (segment (start 139.36 102.6) (end 139.36 102.6385) (width 0.45) (layer B.Cu) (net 5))
 (segment (start 139.92909 103.28959) (end 139.92909 105.2) (width 0.45) (layer F.Cu) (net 5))
 (segment (start 139.319 102.6795) (end 139.92909 103.28959) (width 0.45) (layer F.Cu) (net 5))
 (segment (start 146.315523 95.910499) (end 146.551012 95.67501) (width 0.45) (layer F.Cu) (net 7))
 (segment (start 141.262001 95.910499) (end 146.315523 95.910499) (width 0.45) (layer F.Cu) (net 7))
 (segment (start 141.671501 95.910499) (end 141.262001 95.910499) (width 0.45) (layer F.Cu) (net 7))
 (segment (start 139.845207 95.908099) (end 141.262001 95.908099) (width 0.45) (layer F.Cu) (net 7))
 (segment (start 139.600496 96.15281) (end 139.845207 95.908099) (width 0.45) (layer F.Cu) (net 7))
 (segment (start 139.413836 96.15281) (end 139.600496 96.15281) (width 0.45) (layer F.Cu) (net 7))
 (segment (start 138.6315 96.935146) (end 139.413836 96.15281) (width 0.45) (layer F.Cu) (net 7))
 (segment (start 138.6315 98) (end 138.6315 96.935146) (width 0.45) (layer F.Cu) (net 7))
 (segment (start 137.9815 107.0175) (end 137.811 107.188) (width 0.45) (layer F.Cu) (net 6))
 (segment (start 137.9815 105.1) (end 137.9815 107.0175) (width 0.45) (layer F.Cu) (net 6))
 (via (at 139.5095 107.188) (size 0.8) (drill 0.4) (layers F.Cu B.Cu) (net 12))
 (segment (start 139.5095 107.188) (end 141.415 107.188) (width 0.5) (layer B.Cu) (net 12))
 (segment (start 139.5095 107.188) (end 140.0015 107.188) (width 0.5) (layer F.Cu) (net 12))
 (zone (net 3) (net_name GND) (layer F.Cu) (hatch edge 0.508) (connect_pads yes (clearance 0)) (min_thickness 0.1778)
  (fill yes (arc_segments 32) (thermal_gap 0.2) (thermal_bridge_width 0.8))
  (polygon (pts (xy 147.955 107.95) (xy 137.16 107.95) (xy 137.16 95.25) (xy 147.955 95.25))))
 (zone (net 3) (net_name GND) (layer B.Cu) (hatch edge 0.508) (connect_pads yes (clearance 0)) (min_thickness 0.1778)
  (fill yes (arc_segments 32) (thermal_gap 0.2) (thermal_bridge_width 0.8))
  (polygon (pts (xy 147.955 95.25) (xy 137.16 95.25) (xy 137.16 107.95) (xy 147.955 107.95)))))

